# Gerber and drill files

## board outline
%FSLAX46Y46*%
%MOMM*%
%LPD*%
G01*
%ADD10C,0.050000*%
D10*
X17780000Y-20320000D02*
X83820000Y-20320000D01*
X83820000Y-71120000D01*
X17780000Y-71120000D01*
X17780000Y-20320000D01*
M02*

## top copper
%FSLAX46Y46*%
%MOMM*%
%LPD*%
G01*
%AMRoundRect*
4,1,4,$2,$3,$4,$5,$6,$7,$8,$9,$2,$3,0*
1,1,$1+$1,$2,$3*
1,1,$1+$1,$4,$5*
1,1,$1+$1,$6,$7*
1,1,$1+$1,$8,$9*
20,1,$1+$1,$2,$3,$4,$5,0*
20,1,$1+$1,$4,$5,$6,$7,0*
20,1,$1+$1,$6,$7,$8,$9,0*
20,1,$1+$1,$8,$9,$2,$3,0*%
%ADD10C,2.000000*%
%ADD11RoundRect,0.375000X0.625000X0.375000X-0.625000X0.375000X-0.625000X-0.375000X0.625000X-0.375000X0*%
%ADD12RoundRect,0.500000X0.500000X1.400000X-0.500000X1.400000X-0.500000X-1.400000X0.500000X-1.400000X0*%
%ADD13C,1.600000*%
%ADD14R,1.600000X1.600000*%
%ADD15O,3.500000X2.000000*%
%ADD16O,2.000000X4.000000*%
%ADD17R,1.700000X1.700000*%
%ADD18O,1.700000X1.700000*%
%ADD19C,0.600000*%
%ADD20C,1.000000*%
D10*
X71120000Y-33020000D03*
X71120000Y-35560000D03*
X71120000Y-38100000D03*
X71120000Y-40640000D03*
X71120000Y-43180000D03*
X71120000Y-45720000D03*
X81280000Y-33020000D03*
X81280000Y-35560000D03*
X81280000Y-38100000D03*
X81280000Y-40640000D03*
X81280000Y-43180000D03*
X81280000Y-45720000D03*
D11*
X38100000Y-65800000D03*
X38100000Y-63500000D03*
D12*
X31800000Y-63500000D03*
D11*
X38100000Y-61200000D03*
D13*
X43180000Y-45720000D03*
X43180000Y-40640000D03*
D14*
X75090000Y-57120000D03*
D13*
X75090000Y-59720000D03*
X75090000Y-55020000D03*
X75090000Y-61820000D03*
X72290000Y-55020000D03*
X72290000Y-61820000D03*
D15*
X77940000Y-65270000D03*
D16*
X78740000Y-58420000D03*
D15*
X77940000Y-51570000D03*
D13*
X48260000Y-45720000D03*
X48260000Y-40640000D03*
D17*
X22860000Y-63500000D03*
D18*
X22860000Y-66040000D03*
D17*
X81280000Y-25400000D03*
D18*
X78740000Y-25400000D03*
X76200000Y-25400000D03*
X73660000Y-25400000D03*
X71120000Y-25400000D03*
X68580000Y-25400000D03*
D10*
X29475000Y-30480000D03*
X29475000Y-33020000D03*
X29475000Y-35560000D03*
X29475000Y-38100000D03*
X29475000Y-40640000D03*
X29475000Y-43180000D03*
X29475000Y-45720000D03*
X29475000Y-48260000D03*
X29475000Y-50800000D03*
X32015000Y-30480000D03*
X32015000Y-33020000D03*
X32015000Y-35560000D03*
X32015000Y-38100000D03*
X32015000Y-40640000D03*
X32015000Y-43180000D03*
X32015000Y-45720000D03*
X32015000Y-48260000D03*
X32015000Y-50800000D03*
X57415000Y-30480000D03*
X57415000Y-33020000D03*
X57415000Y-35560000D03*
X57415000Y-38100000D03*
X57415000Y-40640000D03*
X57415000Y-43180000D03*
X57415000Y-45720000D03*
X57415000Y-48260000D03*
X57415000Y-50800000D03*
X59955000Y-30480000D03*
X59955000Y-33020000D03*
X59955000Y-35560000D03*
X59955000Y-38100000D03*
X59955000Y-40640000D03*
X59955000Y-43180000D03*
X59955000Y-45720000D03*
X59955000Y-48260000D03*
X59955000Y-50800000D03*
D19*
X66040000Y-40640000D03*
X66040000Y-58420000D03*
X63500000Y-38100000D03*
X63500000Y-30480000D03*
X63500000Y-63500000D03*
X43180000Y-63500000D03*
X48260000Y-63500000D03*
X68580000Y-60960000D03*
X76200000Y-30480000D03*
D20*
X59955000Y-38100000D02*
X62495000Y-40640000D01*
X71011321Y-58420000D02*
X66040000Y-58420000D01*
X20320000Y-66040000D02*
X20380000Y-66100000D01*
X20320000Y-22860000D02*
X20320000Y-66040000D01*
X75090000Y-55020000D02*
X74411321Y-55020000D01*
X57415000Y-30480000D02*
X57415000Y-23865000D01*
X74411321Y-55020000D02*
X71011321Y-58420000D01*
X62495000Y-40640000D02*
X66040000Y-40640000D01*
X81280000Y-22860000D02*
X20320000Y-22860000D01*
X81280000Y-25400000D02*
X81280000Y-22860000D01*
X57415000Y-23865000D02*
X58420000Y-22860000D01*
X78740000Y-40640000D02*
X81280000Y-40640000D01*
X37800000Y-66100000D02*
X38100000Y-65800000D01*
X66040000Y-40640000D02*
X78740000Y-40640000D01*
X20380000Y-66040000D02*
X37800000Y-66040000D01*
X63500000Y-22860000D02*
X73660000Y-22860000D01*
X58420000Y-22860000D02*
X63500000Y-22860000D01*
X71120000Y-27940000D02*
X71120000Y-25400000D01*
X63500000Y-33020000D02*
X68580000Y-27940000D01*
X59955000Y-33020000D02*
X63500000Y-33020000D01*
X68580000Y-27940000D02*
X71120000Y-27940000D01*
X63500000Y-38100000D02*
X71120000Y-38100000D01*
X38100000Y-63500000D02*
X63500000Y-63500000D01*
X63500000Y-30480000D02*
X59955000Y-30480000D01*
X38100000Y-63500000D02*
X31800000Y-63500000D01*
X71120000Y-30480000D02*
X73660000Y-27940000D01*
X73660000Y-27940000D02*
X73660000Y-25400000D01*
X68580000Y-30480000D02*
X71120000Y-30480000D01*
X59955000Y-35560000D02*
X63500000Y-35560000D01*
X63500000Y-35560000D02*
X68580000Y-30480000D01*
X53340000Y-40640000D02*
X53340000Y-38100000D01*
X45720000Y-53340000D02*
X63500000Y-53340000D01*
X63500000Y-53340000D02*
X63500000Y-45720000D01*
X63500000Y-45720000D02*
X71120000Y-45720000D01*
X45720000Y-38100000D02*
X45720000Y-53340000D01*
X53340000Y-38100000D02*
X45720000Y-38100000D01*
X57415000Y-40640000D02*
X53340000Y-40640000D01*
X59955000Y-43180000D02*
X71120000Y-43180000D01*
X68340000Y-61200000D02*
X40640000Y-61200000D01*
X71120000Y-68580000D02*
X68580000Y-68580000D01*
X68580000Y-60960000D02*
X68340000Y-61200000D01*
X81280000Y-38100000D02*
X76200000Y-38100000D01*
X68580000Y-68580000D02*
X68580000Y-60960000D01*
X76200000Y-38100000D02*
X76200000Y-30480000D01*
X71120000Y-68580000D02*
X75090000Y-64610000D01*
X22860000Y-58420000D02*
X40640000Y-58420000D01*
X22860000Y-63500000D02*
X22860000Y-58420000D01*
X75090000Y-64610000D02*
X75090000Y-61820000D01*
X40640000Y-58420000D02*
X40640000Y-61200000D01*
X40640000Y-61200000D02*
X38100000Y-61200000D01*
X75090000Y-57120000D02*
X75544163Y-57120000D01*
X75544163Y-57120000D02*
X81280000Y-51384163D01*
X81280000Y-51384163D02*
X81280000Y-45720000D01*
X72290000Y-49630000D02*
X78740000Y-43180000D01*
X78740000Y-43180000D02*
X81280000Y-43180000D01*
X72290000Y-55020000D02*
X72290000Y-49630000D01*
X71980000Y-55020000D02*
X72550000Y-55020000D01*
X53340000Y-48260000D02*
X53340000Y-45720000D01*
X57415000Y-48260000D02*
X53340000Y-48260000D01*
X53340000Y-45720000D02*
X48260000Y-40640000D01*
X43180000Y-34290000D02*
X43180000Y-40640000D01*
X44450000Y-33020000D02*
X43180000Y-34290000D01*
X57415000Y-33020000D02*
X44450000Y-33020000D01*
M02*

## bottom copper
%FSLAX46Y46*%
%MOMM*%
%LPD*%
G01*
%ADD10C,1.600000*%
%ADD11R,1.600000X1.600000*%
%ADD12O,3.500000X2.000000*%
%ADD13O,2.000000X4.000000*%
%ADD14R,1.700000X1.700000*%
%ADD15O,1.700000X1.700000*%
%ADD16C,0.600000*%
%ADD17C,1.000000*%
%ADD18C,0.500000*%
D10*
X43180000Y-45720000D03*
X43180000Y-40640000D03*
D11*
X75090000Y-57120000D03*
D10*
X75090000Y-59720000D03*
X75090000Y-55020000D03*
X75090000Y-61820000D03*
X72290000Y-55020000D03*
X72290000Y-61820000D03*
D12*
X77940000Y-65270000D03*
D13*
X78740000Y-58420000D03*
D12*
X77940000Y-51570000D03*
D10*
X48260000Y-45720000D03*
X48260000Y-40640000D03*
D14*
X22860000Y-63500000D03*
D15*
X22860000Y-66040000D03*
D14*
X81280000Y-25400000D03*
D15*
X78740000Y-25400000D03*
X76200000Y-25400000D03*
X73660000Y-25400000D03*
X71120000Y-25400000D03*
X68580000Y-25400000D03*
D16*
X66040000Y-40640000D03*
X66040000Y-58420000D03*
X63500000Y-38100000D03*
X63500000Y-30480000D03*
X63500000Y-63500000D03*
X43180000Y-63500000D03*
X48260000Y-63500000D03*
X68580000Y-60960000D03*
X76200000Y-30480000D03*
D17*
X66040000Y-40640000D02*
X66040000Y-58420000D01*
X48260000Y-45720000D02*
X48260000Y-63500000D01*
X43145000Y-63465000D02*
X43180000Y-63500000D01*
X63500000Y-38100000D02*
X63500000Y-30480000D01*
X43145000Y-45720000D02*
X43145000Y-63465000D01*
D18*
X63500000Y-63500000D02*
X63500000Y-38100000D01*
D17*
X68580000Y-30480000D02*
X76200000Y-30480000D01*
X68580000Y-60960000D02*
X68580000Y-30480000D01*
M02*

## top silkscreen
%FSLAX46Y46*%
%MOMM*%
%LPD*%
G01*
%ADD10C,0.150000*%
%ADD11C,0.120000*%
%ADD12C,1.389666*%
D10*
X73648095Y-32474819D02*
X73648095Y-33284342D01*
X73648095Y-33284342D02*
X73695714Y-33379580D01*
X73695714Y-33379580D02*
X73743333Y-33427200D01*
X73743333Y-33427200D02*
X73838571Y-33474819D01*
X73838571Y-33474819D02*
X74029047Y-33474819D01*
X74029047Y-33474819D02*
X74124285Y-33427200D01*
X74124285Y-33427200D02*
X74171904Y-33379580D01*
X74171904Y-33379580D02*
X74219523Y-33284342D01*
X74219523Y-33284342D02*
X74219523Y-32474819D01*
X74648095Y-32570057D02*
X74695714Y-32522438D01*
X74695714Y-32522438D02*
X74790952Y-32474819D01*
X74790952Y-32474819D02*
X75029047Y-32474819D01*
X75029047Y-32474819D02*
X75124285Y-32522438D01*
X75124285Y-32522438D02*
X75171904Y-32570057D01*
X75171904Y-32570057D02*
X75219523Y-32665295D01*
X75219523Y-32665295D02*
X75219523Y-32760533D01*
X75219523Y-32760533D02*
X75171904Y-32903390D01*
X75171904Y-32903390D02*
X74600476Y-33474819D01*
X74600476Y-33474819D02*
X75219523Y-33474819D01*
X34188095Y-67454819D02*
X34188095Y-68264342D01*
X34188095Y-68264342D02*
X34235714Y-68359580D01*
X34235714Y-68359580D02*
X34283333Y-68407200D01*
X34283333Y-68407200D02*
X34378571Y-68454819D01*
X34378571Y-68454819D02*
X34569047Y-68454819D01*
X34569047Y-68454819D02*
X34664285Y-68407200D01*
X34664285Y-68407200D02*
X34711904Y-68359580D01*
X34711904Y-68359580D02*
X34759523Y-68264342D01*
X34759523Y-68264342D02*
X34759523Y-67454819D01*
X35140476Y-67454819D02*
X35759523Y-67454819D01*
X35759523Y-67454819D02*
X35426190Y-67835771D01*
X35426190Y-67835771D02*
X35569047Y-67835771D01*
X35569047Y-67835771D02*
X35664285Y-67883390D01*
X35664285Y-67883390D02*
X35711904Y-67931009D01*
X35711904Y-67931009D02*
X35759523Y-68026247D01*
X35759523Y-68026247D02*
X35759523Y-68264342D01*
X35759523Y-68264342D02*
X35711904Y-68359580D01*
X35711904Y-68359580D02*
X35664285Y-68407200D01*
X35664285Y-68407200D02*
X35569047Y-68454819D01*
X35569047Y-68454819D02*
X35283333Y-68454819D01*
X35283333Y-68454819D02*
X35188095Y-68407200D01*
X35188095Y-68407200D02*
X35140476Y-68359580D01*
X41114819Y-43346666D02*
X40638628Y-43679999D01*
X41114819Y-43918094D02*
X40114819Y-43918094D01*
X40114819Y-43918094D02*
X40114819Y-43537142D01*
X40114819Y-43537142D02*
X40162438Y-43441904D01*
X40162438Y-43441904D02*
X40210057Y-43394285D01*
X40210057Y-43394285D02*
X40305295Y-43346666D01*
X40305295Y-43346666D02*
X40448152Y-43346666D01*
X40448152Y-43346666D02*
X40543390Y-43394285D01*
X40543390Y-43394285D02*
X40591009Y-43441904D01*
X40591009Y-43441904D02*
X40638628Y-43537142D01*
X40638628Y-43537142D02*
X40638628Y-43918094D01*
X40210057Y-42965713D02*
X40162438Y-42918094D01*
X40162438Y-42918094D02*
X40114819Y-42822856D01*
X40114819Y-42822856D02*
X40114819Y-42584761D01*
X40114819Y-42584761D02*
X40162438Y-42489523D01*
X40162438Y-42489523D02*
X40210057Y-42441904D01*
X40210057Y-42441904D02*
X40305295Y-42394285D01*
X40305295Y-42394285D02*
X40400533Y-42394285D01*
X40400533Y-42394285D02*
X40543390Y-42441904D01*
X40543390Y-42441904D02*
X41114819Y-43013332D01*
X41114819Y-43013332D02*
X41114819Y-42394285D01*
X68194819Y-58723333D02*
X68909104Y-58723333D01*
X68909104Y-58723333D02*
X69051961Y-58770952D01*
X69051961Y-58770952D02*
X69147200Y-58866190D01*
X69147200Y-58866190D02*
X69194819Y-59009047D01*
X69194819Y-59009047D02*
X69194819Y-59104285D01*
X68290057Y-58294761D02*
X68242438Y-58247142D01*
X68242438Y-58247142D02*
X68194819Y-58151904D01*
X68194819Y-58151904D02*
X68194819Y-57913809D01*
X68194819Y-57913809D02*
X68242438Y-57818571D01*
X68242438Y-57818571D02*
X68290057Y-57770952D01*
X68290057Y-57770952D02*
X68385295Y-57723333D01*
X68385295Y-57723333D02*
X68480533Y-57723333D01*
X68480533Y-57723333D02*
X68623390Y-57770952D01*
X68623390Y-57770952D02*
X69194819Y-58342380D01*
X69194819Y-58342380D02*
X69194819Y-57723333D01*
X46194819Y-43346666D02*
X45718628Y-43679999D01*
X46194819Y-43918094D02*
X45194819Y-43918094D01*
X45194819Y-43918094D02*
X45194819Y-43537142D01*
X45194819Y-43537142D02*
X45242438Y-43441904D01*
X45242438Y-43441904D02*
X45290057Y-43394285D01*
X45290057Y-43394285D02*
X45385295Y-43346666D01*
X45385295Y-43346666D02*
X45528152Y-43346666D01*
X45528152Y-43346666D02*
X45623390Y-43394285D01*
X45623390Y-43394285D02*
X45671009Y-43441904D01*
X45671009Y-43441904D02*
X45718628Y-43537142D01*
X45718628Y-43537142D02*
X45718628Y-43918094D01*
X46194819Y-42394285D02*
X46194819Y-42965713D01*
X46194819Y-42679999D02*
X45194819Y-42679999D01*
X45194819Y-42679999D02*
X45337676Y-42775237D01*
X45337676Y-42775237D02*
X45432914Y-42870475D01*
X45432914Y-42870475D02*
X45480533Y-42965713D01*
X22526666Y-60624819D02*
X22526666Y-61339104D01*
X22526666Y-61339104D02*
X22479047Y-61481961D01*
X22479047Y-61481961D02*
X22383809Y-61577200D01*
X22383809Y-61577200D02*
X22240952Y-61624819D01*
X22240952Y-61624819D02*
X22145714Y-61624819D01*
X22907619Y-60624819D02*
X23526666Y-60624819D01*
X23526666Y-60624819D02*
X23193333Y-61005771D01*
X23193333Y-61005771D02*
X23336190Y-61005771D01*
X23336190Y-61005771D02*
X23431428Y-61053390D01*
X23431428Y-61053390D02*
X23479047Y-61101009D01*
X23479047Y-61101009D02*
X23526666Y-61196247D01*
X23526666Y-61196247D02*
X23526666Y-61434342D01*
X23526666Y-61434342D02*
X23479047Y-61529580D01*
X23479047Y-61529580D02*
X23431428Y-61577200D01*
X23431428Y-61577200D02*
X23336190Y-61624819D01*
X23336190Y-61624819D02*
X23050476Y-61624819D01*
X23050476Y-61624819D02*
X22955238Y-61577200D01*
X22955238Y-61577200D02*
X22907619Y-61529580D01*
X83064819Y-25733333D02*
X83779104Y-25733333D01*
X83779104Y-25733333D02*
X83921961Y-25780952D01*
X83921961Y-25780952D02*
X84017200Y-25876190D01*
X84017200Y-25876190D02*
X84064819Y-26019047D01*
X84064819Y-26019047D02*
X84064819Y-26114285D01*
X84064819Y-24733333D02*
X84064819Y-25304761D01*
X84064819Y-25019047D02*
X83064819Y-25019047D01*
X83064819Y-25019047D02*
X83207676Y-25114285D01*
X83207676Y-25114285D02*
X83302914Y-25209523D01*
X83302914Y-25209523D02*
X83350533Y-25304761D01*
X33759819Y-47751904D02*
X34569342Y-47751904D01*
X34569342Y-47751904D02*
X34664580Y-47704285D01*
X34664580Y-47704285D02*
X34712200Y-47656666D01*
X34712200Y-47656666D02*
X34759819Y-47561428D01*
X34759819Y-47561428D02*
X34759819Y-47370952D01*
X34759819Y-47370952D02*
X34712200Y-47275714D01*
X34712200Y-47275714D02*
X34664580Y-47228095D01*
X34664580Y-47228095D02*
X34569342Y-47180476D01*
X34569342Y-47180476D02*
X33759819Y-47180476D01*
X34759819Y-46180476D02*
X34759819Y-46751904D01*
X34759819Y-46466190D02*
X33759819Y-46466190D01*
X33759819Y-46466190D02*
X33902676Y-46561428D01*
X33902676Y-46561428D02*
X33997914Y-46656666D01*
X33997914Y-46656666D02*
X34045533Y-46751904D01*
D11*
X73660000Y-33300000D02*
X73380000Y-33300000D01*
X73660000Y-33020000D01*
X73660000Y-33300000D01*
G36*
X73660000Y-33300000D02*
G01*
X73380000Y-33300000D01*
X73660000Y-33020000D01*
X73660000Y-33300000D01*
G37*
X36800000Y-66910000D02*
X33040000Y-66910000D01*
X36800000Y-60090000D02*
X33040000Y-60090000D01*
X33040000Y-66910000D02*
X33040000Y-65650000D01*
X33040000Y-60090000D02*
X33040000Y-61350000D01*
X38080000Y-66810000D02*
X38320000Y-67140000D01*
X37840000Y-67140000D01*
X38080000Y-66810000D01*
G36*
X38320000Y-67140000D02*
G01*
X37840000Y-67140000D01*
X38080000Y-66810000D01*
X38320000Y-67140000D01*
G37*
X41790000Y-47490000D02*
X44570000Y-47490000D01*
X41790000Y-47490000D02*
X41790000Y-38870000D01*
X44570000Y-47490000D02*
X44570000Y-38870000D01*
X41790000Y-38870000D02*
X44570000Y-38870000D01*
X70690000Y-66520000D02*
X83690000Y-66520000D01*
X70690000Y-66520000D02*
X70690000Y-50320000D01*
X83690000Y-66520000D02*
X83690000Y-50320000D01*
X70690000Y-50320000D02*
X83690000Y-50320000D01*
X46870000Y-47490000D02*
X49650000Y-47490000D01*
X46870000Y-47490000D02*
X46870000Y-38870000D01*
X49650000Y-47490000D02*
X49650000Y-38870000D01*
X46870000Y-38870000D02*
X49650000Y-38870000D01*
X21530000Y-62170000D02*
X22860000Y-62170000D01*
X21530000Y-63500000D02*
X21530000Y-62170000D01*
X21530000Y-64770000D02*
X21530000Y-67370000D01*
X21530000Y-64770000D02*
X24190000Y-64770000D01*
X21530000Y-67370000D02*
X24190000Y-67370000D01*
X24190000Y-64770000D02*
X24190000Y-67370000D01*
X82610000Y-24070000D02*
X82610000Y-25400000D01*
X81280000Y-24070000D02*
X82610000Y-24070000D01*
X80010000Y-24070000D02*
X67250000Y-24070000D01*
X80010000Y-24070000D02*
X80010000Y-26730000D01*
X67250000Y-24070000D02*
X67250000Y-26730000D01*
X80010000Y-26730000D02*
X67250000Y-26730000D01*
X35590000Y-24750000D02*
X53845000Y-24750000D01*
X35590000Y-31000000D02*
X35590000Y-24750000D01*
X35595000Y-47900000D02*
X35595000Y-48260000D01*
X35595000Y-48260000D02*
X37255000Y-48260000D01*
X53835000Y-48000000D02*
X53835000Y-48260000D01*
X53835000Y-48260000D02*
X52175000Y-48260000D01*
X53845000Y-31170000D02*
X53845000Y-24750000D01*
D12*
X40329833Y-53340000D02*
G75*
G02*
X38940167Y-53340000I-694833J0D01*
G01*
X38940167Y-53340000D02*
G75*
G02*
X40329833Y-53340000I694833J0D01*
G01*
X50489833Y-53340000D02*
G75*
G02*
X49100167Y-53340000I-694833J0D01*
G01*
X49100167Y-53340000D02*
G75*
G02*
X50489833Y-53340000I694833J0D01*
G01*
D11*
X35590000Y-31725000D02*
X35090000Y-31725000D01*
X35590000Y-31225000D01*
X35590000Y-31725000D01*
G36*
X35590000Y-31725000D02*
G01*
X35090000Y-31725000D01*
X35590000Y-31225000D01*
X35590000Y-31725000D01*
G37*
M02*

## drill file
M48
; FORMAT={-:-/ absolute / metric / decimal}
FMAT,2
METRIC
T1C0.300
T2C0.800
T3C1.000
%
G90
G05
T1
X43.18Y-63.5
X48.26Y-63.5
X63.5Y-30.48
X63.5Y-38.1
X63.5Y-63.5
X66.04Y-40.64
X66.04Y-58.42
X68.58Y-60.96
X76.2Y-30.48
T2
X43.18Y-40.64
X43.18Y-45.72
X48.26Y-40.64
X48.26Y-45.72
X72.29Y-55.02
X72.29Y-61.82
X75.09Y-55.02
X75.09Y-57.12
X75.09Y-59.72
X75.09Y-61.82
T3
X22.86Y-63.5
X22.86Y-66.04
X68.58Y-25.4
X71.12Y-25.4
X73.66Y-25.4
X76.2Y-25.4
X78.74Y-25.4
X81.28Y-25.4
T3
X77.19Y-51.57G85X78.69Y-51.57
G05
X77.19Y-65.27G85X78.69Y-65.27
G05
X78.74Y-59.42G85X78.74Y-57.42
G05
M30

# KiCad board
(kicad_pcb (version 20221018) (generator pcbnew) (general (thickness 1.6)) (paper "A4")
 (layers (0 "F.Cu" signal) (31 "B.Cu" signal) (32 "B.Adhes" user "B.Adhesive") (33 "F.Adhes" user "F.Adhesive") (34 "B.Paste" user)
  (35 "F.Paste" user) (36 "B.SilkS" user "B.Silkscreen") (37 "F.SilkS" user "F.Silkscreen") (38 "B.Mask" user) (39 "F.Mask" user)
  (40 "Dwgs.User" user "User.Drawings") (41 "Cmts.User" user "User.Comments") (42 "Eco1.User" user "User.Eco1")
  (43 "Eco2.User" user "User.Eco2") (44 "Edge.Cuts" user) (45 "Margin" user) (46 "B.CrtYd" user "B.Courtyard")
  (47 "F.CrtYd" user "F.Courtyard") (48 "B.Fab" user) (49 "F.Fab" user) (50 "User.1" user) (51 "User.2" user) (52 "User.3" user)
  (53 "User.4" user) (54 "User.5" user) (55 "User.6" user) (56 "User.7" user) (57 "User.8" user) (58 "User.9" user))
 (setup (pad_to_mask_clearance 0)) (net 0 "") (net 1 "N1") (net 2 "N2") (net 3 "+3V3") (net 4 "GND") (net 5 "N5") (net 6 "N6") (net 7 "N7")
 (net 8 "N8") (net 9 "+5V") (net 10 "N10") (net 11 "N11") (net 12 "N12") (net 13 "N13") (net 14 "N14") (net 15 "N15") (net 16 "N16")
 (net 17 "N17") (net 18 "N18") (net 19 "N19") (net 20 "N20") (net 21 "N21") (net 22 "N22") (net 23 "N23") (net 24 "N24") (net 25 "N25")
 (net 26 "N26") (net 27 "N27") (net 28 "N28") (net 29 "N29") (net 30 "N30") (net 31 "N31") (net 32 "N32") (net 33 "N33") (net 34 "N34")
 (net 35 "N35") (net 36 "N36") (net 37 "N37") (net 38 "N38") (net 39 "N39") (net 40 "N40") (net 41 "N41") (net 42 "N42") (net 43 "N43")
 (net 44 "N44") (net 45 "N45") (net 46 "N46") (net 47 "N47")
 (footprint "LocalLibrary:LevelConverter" (layer "F.Cu") (at 76.2 38.1)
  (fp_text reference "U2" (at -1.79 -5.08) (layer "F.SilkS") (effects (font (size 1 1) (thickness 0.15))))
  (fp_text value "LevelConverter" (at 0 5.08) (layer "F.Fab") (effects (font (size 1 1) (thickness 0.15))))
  (fp_poly
   (pts (xy -2.54 -4.8) (xy -2.82 -4.8) (xy -2.54 -5.08) (xy -2.54 -4.8)) (stroke (width 0.12) (type solid)) (fill solid) (layer "F.SilkS"))
  (pad "1" smd circle (at -5.08 -5.08 270) (size 2 2) (layers "F.Cu" "F.Paste" "F.Mask") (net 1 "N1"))
  (pad "2" smd circle (at -5.08 -2.54 270) (size 2 2) (layers "F.Cu" "F.Paste" "F.Mask") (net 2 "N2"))
  (pad "3" smd circle (at -5.08 0 270) (size 2 2) (layers "F.Cu" "F.Paste" "F.Mask") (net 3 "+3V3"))
  (pad "4" smd circle (at -5.08 2.54 270) (size 2 2) (layers "F.Cu" "F.Paste" "F.Mask") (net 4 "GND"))
  (pad "5" smd circle (at -5.08 5.08 270) (size 2 2) (layers "F.Cu" "F.Paste" "F.Mask") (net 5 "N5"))
  (pad "6" smd circle (at -5.08 7.62 270) (size 2 2) (layers "F.Cu" "F.Paste" "F.Mask") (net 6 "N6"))
  (pad "7" smd circle (at 5.08 -5.08 270) (size 2 2) (layers "F.Cu" "F.Paste" "F.Mask") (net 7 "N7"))
  (pad "8" smd circle (at 5.08 -2.54 270) (size 2 2) (layers "F.Cu" "F.Paste" "F.Mask") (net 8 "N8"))
  (pad "9" smd circle (at 5.08 0 270) (size 2 2) (layers "F.Cu" "F.Paste" "F.Mask") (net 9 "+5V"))
  (pad "10" smd circle (at 5.08 2.54 270) (size 2 2) (layers "F.Cu" "F.Paste" "F.Mask") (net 4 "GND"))
  (pad "11" smd circle (at 5.08 5.08) (size 2 2) (layers "F.Cu" "F.Paste" "F.Mask") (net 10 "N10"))
  (pad "12" smd circle (at 5.08 7.62) (size 2 2) (layers "F.Cu" "F.Paste" "F.Mask") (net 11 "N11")))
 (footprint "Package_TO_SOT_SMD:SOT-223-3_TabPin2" (layer "F.Cu") (at 34.95 63.5 180)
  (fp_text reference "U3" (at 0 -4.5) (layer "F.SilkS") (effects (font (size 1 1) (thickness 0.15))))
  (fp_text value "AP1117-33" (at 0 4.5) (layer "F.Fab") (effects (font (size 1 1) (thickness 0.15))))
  (fp_line (start -1.85 -3.41) (end 1.91 -3.41) (stroke (width 0.12) (type solid)) (layer "F.SilkS"))
  (fp_line (start -1.85 3.41) (end 1.91 3.41) (stroke (width 0.12) (type solid)) (layer "F.SilkS"))
  (fp_line (start 1.91 -3.41) (end 1.91 -2.15) (stroke (width 0.12) (type solid)) (layer "F.SilkS"))
  (fp_line (start 1.91 3.41) (end 1.91 2.15) (stroke (width 0.12) (type solid)) (layer "F.SilkS"))
  (fp_poly
   (pts (xy -3.13 -3.31) (xy -3.37 -3.64) (xy -2.89 -3.64) (xy -3.13 -3.31)) (stroke (width 0.12) (type solid)) (fill solid)
   (layer "F.SilkS"))
  (pad "1" smd roundrect (at -3.15 -2.3 180) (size 2 1.5) (layers "F.Cu" "F.Paste" "F.Mask") (roundrect_rratio 0.25) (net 4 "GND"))
  (pad "2" smd roundrect (at -3.15 0 180) (size 2 1.5) (layers "F.Cu" "F.Paste" "F.Mask") (roundrect_rratio 0.25) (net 3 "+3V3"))
  (pad "2" smd roundrect (at 3.15 0 180) (size 2 3.8) (layers "F.Cu" "F.Paste" "F.Mask") (roundrect_rratio 0.25) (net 3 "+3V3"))
  (pad "3" smd roundrect (at -3.15 2.3 180) (size 2 1.5) (layers "F.Cu" "F.Paste" "F.Mask") (roundrect_rratio 0.25) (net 9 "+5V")))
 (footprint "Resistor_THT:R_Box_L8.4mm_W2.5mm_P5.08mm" (layer "F.Cu") (at 43.18 45.72 90)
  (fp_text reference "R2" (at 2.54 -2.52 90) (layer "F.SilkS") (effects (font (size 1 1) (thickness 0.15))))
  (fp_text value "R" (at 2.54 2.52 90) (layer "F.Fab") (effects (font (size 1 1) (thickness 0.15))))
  (fp_line (start -1.77 -1.39) (end -1.77 1.39) (stroke (width 0.12) (type solid)) (layer "F.SilkS"))
  (fp_line (start -1.77 -1.39) (end 6.85 -1.39) (stroke (width 0.12) (type solid)) (layer "F.SilkS"))
  (fp_line (start -1.77 1.39) (end 6.85 1.39) (stroke (width 0.12) (type solid)) (layer "F.SilkS"))
  (fp_line (start 6.85 -1.39) (end 6.85 1.39) (stroke (width 0.12) (type solid)) (layer "F.SilkS"))
  (pad "1" thru_hole circle (at 0 0 90) (size 1.6 1.6) (drill 0.8) (layers "*.Cu" "*.Mask") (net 3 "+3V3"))
  (pad "2" thru_hole circle (at 5.08 0 90) (size 1.6 1.6) (drill 0.8) (layers "*.Cu" "*.Mask") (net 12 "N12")))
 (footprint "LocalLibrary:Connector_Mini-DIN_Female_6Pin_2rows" (layer "F.Cu") (at 75.09 57.12 90)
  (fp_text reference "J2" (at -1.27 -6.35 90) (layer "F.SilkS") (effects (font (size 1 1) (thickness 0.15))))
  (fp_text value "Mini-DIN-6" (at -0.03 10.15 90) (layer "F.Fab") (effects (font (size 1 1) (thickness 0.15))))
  (fp_line (start -9.4 -4.4) (end -9.4 8.6) (stroke (width 0.12) (type solid)) (layer "F.SilkS"))
  (fp_line (start -9.4 -4.4) (end 6.8 -4.4) (stroke (width 0.12) (type solid)) (layer "F.SilkS"))
  (fp_line (start -9.4 8.6) (end 6.8 8.6) (stroke (width 0.12) (type solid)) (layer "F.SilkS"))
  (fp_line (start 6.8 -4.4) (end 6.8 8.6) (stroke (width 0.12) (type solid)) (layer "F.SilkS"))
  (pad "1" thru_hole rect (at 0 0 90) (size 1.6 1.6) (drill 0.8) (layers "*.Cu" "*.Mask") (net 11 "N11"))
  (pad "2" thru_hole circle (at -2.6 0 90) (size 1.6 1.6) (drill 0.8) (layers "*.Cu" "*.Mask") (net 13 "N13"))
  (pad "3" thru_hole circle (at 2.1 0 90) (size 1.6 1.6) (drill 0.8) (layers "*.Cu" "*.Mask") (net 4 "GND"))
  (pad "4" thru_hole circle (at -4.7 0 90) (size 1.6 1.6) (drill 0.8) (layers "*.Cu" "*.Mask") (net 9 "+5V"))
  (pad "5" thru_hole circle (at 2.1 -2.8 90) (size 1.6 1.6) (drill 0.8) (layers "*.Cu" "*.Mask") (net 10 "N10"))
  (pad "6" thru_hole circle (at -4.7 -2.8 90) (size 1.6 1.6) (drill 0.8) (layers "*.Cu" "*.Mask") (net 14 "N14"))
  (pad "7" thru_hole oval (at -8.15 2.85 90) (size 2 3.5) (drill oval 1 2.5) (layers "*.Cu" "*.Mask"))
  (pad "7" thru_hole oval (at -1.3 3.65 90) (size 4 2) (drill oval 3 1) (layers "*.Cu" "*.Mask"))
  (pad "7" thru_hole oval (at 5.55 2.85 90) (size 2 3.5) (drill oval 1 2.5) (layers "*.Cu" "*.Mask")))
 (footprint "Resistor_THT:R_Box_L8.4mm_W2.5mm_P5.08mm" (layer "F.Cu") (at 48.26 45.72 90)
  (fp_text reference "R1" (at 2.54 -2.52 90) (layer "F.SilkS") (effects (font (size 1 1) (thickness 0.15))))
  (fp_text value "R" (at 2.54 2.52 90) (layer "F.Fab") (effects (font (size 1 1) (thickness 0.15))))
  (fp_line (start -1.77 -1.39) (end -1.77 1.39) (stroke (width 0.12) (type solid)) (layer "F.SilkS"))
  (fp_line (start -1.77 -1.39) (end 6.85 -1.39) (stroke (width 0.12) (type solid)) (layer "F.SilkS"))
  (fp_line (start -1.77 1.39) (end 6.85 1.39) (stroke (width 0.12) (type solid)) (layer "F.SilkS"))
  (fp_line (start 6.85 -1.39) (end 6.85 1.39) (stroke (width 0.12) (type solid)) (layer "F.SilkS"))
  (pad "1" thru_hole circle (at 0 0 90) (size 1.6 1.6) (drill 0.8) (layers "*.Cu" "*.Mask") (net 3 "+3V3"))
  (pad "2" thru_hole circle (at 5.08 0 90) (size 1.6 1.6) (drill 0.8) (layers "*.Cu" "*.Mask") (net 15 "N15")))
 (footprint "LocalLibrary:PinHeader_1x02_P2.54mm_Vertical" (layer "F.Cu") (at 22.86 63.5)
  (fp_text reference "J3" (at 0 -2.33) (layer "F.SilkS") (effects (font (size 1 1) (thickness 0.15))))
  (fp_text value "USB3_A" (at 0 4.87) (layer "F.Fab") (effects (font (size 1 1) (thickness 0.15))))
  (fp_line (start -1.33 -1.33) (end 0 -1.33) (stroke (width 0.12) (type solid)) (layer "F.SilkS"))
  (fp_line (start -1.33 0) (end -1.33 -1.33) (stroke (width 0.12) (type solid)) (layer "F.SilkS"))
  (fp_line (start -1.33 1.27) (end -1.33 3.87) (stroke (width 0.12) (type solid)) (layer "F.SilkS"))
  (fp_line (start -1.33 1.27) (end 1.33 1.27) (stroke (width 0.12) (type solid)) (layer "F.SilkS"))
  (fp_line (start -1.33 3.87) (end 1.33 3.87) (stroke (width 0.12) (type solid)) (layer "F.SilkS"))
  (fp_line (start 1.33 1.27) (end 1.33 3.87) (stroke (width 0.12) (type solid)) (layer "F.SilkS"))
  (pad "1" thru_hole rect (at 0 0) (size 1.7 1.7) (drill 1) (layers "*.Cu" "*.Mask") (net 9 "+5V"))
  (pad "4" thru_hole oval (at 0 2.54) (size 1.7 1.7) (drill 1) (layers "*.Cu" "*.Mask") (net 4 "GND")))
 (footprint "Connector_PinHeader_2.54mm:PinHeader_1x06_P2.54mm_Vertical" (layer "F.Cu") (at 81.28 25.4 -90)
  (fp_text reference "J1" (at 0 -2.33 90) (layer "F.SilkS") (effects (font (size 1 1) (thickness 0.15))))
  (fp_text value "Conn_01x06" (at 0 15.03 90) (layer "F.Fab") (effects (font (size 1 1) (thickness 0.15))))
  (fp_line (start -1.33 -1.33) (end 0 -1.33) (stroke (width 0.12) (type solid)) (layer "F.SilkS"))
  (fp_line (start -1.33 0) (end -1.33 -1.33) (stroke (width 0.12) (type solid)) (layer "F.SilkS"))
  (fp_line (start -1.33 1.27) (end -1.33 14.03) (stroke (width 0.12) (type solid)) (layer "F.SilkS"))
  (fp_line (start -1.33 1.27) (end 1.33 1.27) (stroke (width 0.12) (type solid)) (layer "F.SilkS"))
  (fp_line (start -1.33 14.03) (end 1.33 14.03) (stroke (width 0.12) (type solid)) (layer "F.SilkS"))
  (fp_line (start 1.33 1.27) (end 1.33 14.03) (stroke (width 0.12) (type solid)) (layer "F.SilkS"))
  (pad "1" thru_hole rect (at 0 0 270) (size 1.7 1.7) (drill 1) (layers "*.Cu" "*.Mask") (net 4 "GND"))
  (pad "2" thru_hole oval (at 0 2.54 270) (size 1.7 1.7) (drill 1) (layers "*.Cu" "*.Mask") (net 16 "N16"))
  (pad "3" thru_hole oval (at 0 5.08 270) (size 1.7 1.7) (drill 1) (layers "*.Cu" "*.Mask") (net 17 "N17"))
  (pad "4" thru_hole oval (at 0 7.62 270) (size 1.7 1.7) (drill 1) (layers "*.Cu" "*.Mask") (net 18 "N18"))
  (pad "5" thru_hole oval (at 0 10.16 270) (size 1.7 1.7) (drill 1) (layers "*.Cu" "*.Mask") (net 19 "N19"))
  (pad "6" thru_hole oval (at 0 12.7 270) (size 1.7 1.7) (drill 1) (layers "*.Cu" "*.Mask") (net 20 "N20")))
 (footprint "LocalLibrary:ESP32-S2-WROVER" (layer "F.Cu") (at 44.715 40.64)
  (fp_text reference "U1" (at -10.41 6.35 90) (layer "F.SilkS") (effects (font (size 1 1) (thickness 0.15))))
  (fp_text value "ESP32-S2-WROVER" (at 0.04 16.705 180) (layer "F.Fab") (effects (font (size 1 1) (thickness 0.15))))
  (fp_line (start -9.125 -15.89) (end 9.13 -15.89) (stroke (width 0.12) (type solid)) (layer "F.SilkS"))
  (fp_line (start -9.125 -9.64) (end -9.125 -15.89) (stroke (width 0.12) (type solid)) (layer "F.SilkS"))
  (fp_line (start -9.12 7.26) (end -9.12 7.62) (stroke (width 0.12) (type solid)) (layer "F.SilkS"))
  (fp_line (start -9.12 7.62) (end -7.46 7.62) (stroke (width 0.12) (type solid)) (layer "F.SilkS"))
  (fp_line (start 9.12 7.36) (end 9.12 7.62) (stroke (width 0.12) (type solid)) (layer "F.SilkS"))
  (fp_line (start 9.12 7.62) (end 7.46 7.62) (stroke (width 0.12) (type solid)) (layer "F.SilkS"))
  (fp_line (start 9.13 -9.47) (end 9.13 -15.89) (stroke (width 0.12) (type solid)) (layer "F.SilkS"))
  (fp_circle (center -5.08 12.7) (end -3.740334 12.7) (stroke (width 0.1) (type solid)) (fill solid) (layer "F.SilkS"))
  (fp_circle (center 5.08 12.7) (end 6.419666 12.7) (stroke (width 0.1) (type solid)) (fill solid) (layer "F.SilkS"))
  (fp_poly
   (pts (xy -9.125 -8.915) (xy -9.625 -8.915) (xy -9.125 -9.415) (xy -9.125 -8.915)) (stroke (width 0.12) (type solid)) (fill solid)
   (layer "F.SilkS"))
  (pad "1" smd circle (at -15.24 -10.16) (size 2 2) (layers "F.Cu" "F.Paste" "F.Mask") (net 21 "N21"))
  (pad "2" smd circle (at -15.24 -7.62) (size 2 2) (layers "F.Cu" "F.Paste" "F.Mask") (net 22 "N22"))
  (pad "3" smd circle (at -15.24 -5.08) (size 2 2) (layers "F.Cu" "F.Paste" "F.Mask") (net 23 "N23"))
  (pad "4" smd circle (at -15.24 -2.54) (size 2 2) (layers "F.Cu" "F.Paste" "F.Mask") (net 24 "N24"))
  (pad "5" smd circle (at -15.24 0) (size 2 2) (layers "F.Cu" "F.Paste" "F.Mask") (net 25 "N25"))
  (pad "6" smd circle (at -15.24 2.54) (size 2 2) (layers "F.Cu" "F.Paste" "F.Mask") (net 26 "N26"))
  (pad "7" smd circle (at -15.24 5.08) (size 2 2) (layers "F.Cu" "F.Paste" "F.Mask") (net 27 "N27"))
  (pad "8" smd circle (at -15.24 7.62) (size 2 2) (layers "F.Cu" "F.Paste" "F.Mask") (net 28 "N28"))
  (pad "9" smd circle (at -15.24 10.16) (size 2 2) (layers "F.Cu" "F.Paste" "F.Mask") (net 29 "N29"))
  (pad "10" smd circle (at -12.7 -10.16) (size 2 2) (layers "F.Cu" "F.Paste" "F.Mask") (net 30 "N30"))
  (pad "11" smd circle (at -12.7 -7.62) (size 2 2) (layers "F.Cu" "F.Paste" "F.Mask") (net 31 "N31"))
  (pad "12" smd circle (at -12.7 -5.08) (size 2 2) (layers "F.Cu" "F.Paste" "F.Mask") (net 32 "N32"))
  (pad "13" smd circle (at -12.7 -2.54) (size 2 2) (layers "F.Cu" "F.Paste" "F.Mask") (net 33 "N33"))
  (pad "14" smd circle (at -12.7 0) (size 2 2) (layers "F.Cu" "F.Paste" "F.Mask") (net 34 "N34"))
  (pad "15" smd circle (at -12.7 2.54) (size 2 2) (layers "F.Cu" "F.Paste" "F.Mask") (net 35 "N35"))
  (pad "16" smd circle (at -12.7 5.08) (size 2 2) (layers "F.Cu" "F.Paste" "F.Mask") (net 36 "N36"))
  (pad "17" smd circle (at -12.7 7.62) (size 2 2) (layers "F.Cu" "F.Paste" "F.Mask") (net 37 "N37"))
  (pad "18" smd circle (at -12.7 10.16) (size 2 2) (layers "F.Cu" "F.Paste" "F.Mask") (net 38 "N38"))
  (pad "19" smd circle (at 12.7 -10.16) (size 2 2) (layers "F.Cu" "F.Paste" "F.Mask") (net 4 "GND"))
  (pad "20" smd circle (at 12.7 -7.62) (size 2 2) (layers "F.Cu" "F.Paste" "F.Mask") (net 12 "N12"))
  (pad "21" smd circle (at 12.7 -5.08) (size 2 2) (layers "F.Cu" "F.Paste" "F.Mask") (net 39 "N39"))
  (pad "22" smd circle (at 12.7 -2.54) (size 2 2) (layers "F.Cu" "F.Paste" "F.Mask") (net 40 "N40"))
  (pad "23" smd circle (at 12.7 0) (size 2 2) (layers "F.Cu" "F.Paste" "F.Mask") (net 6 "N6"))
  (pad "24" smd circle (at 12.7 2.54) (size 2 2) (layers "F.Cu" "F.Paste" "F.Mask") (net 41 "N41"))
  (pad "25" smd circle (at 12.7 5.08) (size 2 2) (layers "F.Cu" "F.Paste" "F.Mask") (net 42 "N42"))
  (pad "26" smd circle (at 12.7 7.62) (size 2 2) (layers "F.Cu" "F.Paste" "F.Mask") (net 15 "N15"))
  (pad "27" smd circle (at 12.7 10.16) (size 2 2) (layers "F.Cu" "F.Paste" "F.Mask") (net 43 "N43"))
  (pad "28" smd circle (at 15.24 -10.16) (size 2 2) (layers "F.Cu" "F.Paste" "F.Mask") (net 3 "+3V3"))
  (pad "29" smd circle (at 15.24 -7.62) (size 2 2) (layers "F.Cu" "F.Paste" "F.Mask") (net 19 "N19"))
  (pad "30" smd circle (at 15.24 -5.08) (size 2 2) (layers "F.Cu" "F.Paste" "F.Mask") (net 18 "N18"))
  (pad "31" smd circle (at 15.24 -2.54) (size 2 2) (layers "F.Cu" "F.Paste" "F.Mask") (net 4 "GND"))
  (pad "32" smd circle (at 15.24 0) (size 2 2) (layers "F.Cu" "F.Paste" "F.Mask") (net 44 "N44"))
  (pad "33" smd circle (at 15.24 2.54) (size 2 2) (layers "F.Cu" "F.Paste" "F.Mask") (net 5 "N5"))
  (pad "34" smd circle (at 15.24 5.08) (size 2 2) (layers "F.Cu" "F.Paste" "F.Mask") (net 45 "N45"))
  (pad "35" smd circle (at 15.24 7.62) (size 2 2) (layers "F.Cu" "F.Paste" "F.Mask") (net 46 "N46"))
  (pad "36" smd circle (at 15.24 10.16) (size 2 2) (layers "F.Cu" "F.Paste" "F.Mask") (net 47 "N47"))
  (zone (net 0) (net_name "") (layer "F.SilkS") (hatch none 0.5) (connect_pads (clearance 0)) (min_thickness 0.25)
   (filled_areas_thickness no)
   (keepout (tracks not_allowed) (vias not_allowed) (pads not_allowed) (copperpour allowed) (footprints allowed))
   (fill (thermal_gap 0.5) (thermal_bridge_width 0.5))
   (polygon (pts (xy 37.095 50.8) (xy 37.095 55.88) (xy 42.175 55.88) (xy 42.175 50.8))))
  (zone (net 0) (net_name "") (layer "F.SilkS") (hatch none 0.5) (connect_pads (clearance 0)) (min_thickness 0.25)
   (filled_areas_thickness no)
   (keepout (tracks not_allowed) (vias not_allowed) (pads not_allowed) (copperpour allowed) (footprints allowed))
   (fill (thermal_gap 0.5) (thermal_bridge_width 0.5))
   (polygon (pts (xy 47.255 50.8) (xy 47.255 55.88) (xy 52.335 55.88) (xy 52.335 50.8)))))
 (gr_rect (start 17.78 20.32) (end 83.82 71.12) (stroke (width 0.05) (type default)) (fill none) (layer "Edge.Cuts"))
 (segment (start 59.955 38.1) (end 62.495 40.64) (width 1) (layer "F.Cu") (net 4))
 (segment (start 71.011321 58.42) (end 66.04 58.42) (width 1) (layer "F.Cu") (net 4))
 (segment (start 20.32 66.04) (end 20.38 66.1) (width 1) (layer "F.Cu") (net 4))
 (segment (start 20.32 22.86) (end 20.32 66.04) (width 1) (layer "F.Cu") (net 4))
 (segment (start 75.09 55.02) (end 74.411321 55.02) (width 1) (layer "F.Cu") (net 4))
 (segment (start 57.415 30.48) (end 57.415 23.865) (width 1) (layer "F.Cu") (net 4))
 (segment (start 74.411321 55.02) (end 71.011321 58.42) (width 1) (layer "F.Cu") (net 4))
 (segment (start 62.495 40.64) (end 66.04 40.64) (width 1) (layer "F.Cu") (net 4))
 (segment (start 81.28 22.86) (end 20.32 22.86) (width 1) (layer "F.Cu") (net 4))
 (segment (start 81.28 25.4) (end 81.28 22.86) (width 1) (layer "F.Cu") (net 4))
 (segment (start 57.415 23.865) (end 58.42 22.86) (width 1) (layer "F.Cu") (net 4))
 (segment (start 78.74 40.64) (end 81.28 40.64) (width 1) (layer "F.Cu") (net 4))
 (segment (start 37.8 66.1) (end 38.1 65.8) (width 1) (layer "F.Cu") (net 4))
 (segment (start 66.04 40.64) (end 78.74 40.64) (width 1) (layer "F.Cu") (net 4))
 (segment (start 20.38 66.04) (end 37.8 66.04) (width 1) (layer "F.Cu") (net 4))
 (segment (start 63.5 22.86) (end 73.66 22.86) (width 1) (layer "F.Cu") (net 4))
 (segment (start 58.42 22.86) (end 63.5 22.86) (width 1) (layer "F.Cu") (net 4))
 (via (at 66.04 40.64) (size 0.6) (drill 0.3) (layers "F.Cu" "B.Cu") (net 4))
 (via (at 66.04 58.42) (size 0.6) (drill 0.3) (layers "F.Cu" "B.Cu") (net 4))
 (segment (start 66.04 40.64) (end 66.04 58.42) (width 1) (layer "B.Cu") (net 4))
 (segment (start 71.12 27.94) (end 71.12 25.4) (width 1) (layer "F.Cu") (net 19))
 (segment (start 63.5 33.02) (end 68.58 27.94) (width 1) (layer "F.Cu") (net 19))
 (segment (start 59.955 33.02) (end 63.5 33.02) (width 1) (layer "F.Cu") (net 19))
 (segment (start 68.58 27.94) (end 71.12 27.94) (width 1) (layer "F.Cu") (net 19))
 (segment (start 63.5 38.1) (end 71.12 38.1) (width 1) (layer "F.Cu") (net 3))
 (segment (start 38.1 63.5) (end 63.5 63.5) (width 1) (layer "F.Cu") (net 3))
 (segment (start 63.5 30.48) (end 59.955 30.48) (width 1) (layer "F.Cu") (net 3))
 (segment (start 38.1 63.5) (end 31.8 63.5) (width 1) (layer "F.Cu") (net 3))
 (via (at 63.5 38.1) (size 0.6) (drill 0.3) (layers "F.Cu" "B.Cu") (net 3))
 (via (at 63.5 30.48) (size 0.6) (drill 0.3) (layers "F.Cu" "B.Cu") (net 3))
 (via (at 63.5 63.5) (size 0.6) (drill 0.3) (layers "F.Cu" "B.Cu") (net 3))
 (via (at 43.18 63.5) (size 0.6) (drill 0.3) (layers "F.Cu" "B.Cu") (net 3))
 (via (at 48.26 63.5) (size 0.6) (drill 0.3) (layers "F.Cu" "B.Cu") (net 3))
 (segment (start 48.26 45.72) (end 48.26 63.5) (width 1) (layer "B.Cu") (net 3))
 (segment (start 43.145 63.465) (end 43.18 63.5) (width 1) (layer "B.Cu") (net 3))
 (segment (start 63.5 38.1) (end 63.5 30.48) (width 1) (layer "B.Cu") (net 3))
 (segment (start 43.145 45.72) (end 43.145 63.465) (width 1) (layer "B.Cu") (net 3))
 (segment (start 63.5 63.5) (end 63.5 38.1) (width 0.5) (layer "B.Cu") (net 3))
 (segment (start 71.12 30.48) (end 73.66 27.94) (width 1) (layer "F.Cu") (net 18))
 (segment (start 73.66 27.94) (end 73.66 25.4) (width 1) (layer "F.Cu") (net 18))
 (segment (start 68.58 30.48) (end 71.12 30.48) (width 1) (layer "F.Cu") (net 18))
 (segment (start 59.955 35.56) (end 63.5 35.56) (width 1) (layer "F.Cu") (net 18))
 (segment (start 63.5 35.56) (end 68.58 30.48) (width 1) (layer "F.Cu") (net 18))
 (segment (start 53.34 40.64) (end 53.34 38.1) (width 1) (layer "F.Cu") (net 6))
 (segment (start 45.72 53.34) (end 63.5 53.34) (width 1) (layer "F.Cu") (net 6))
 (segment (start 63.5 53.34) (end 63.5 45.72) (width 1) (layer "F.Cu") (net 6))
 (segment (start 63.5 45.72) (end 71.12 45.72) (width 1) (layer "F.Cu") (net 6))
 (segment (start 45.72 38.1) (end 45.72 53.34) (width 1) (layer "F.Cu") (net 6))
 (segment (start 53.34 38.1) (end 45.72 38.1) (width 1) (layer "F.Cu") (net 6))
 (segment (start 57.415 40.64) (end 53.34 40.64) (width 1) (layer "F.Cu") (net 6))
 (segment (start 59.955 43.18) (end 71.12 43.18) (width 1) (layer "F.Cu") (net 5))
 (segment (start 68.34 61.2) (end 40.64 61.2) (width 1) (layer "F.Cu") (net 9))
 (segment (start 71.12 68.58) (end 68.58 68.58) (width 1) (layer "F.Cu") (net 9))
 (segment (start 68.58 60.96) (end 68.34 61.2) (width 1) (layer "F.Cu") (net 9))
 (segment (start 81.28 38.1) (end 76.2 38.1) (width 1) (layer "F.Cu") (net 9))
 (segment (start 68.58 68.58) (end 68.58 60.96) (width 1) (layer "F.Cu") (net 9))
 (segment (start 76.2 38.1) (end 76.2 30.48) (width 1) (layer "F.Cu") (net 9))
 (segment (start 71.12 68.58) (end 75.09 64.61) (width 1) (layer "F.Cu") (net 9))
 (segment (start 22.86 58.42) (end 40.64 58.42) (width 1) (layer "F.Cu") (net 9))
 (segment (start 22.86 63.5) (end 22.86 58.42) (width 1) (layer "F.Cu") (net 9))
 (segment (start 75.09 64.61) (end 75.09 61.82) (width 1) (layer "F.Cu") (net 9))
 (segment (start 40.64 58.42) (end 40.64 61.2) (width 1) (layer "F.Cu") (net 9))
 (segment (start 40.64 61.2) (end 38.1 61.2) (width 1) (layer "F.Cu") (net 9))
 (via (at 68.58 60.96) (size 0.6) (drill 0.3) (layers "F.Cu" "B.Cu") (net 9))
 (via (at 76.2 30.48) (size 0.6) (drill 0.3) (layers "F.Cu" "B.Cu") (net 9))
 (segment (start 68.58 30.48) (end 76.2 30.48) (width 1) (layer "B.Cu") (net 9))
 (segment (start 68.58 60.96) (end 68.58 30.48) (width 1) (layer "B.Cu") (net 9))
 (segment (start 75.09 57.12) (end 75.544163 57.12) (width 1) (layer "F.Cu") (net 11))
 (segment (start 75.544163 57.12) (end 81.28 51.384163) (width 1) (layer "F.Cu") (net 11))
 (segment (start 81.28 51.384163) (end 81.28 45.72) (width 1) (layer "F.Cu") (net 11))
 (segment (start 72.29 49.63) (end 78.74 43.18) (width 1) (layer "F.Cu") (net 10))
 (segment (start 78.74 43.18) (end 81.28 43.18) (width 1) (layer "F.Cu") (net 10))
 (segment (start 72.29 55.02) (end 72.29 49.63) (width 1) (layer "F.Cu") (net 10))
 (segment (start 71.98 55.02) (end 72.55 55.02) (width 1) (layer "F.Cu") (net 10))
 (segment (start 53.34 48.26) (end 53.34 45.72) (width 1) (layer "F.Cu") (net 15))
 (segment (start 57.415 48.26) (end 53.34 48.26) (width 1) (layer "F.Cu") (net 15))
 (segment (start 53.34 45.72) (end 48.26 40.64) (width 1) (layer "F.Cu") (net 15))
 (segment (start 43.18 34.29) (end 43.18 40.64) (width 1) (layer "F.Cu") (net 12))
 (segment (start 44.45 33.02) (end 43.18 34.29) (width 1) (layer "F.Cu") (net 12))
 (segment (start 57.415 33.02) (end 44.45 33.02) (width 1) (layer "F.Cu") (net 12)))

